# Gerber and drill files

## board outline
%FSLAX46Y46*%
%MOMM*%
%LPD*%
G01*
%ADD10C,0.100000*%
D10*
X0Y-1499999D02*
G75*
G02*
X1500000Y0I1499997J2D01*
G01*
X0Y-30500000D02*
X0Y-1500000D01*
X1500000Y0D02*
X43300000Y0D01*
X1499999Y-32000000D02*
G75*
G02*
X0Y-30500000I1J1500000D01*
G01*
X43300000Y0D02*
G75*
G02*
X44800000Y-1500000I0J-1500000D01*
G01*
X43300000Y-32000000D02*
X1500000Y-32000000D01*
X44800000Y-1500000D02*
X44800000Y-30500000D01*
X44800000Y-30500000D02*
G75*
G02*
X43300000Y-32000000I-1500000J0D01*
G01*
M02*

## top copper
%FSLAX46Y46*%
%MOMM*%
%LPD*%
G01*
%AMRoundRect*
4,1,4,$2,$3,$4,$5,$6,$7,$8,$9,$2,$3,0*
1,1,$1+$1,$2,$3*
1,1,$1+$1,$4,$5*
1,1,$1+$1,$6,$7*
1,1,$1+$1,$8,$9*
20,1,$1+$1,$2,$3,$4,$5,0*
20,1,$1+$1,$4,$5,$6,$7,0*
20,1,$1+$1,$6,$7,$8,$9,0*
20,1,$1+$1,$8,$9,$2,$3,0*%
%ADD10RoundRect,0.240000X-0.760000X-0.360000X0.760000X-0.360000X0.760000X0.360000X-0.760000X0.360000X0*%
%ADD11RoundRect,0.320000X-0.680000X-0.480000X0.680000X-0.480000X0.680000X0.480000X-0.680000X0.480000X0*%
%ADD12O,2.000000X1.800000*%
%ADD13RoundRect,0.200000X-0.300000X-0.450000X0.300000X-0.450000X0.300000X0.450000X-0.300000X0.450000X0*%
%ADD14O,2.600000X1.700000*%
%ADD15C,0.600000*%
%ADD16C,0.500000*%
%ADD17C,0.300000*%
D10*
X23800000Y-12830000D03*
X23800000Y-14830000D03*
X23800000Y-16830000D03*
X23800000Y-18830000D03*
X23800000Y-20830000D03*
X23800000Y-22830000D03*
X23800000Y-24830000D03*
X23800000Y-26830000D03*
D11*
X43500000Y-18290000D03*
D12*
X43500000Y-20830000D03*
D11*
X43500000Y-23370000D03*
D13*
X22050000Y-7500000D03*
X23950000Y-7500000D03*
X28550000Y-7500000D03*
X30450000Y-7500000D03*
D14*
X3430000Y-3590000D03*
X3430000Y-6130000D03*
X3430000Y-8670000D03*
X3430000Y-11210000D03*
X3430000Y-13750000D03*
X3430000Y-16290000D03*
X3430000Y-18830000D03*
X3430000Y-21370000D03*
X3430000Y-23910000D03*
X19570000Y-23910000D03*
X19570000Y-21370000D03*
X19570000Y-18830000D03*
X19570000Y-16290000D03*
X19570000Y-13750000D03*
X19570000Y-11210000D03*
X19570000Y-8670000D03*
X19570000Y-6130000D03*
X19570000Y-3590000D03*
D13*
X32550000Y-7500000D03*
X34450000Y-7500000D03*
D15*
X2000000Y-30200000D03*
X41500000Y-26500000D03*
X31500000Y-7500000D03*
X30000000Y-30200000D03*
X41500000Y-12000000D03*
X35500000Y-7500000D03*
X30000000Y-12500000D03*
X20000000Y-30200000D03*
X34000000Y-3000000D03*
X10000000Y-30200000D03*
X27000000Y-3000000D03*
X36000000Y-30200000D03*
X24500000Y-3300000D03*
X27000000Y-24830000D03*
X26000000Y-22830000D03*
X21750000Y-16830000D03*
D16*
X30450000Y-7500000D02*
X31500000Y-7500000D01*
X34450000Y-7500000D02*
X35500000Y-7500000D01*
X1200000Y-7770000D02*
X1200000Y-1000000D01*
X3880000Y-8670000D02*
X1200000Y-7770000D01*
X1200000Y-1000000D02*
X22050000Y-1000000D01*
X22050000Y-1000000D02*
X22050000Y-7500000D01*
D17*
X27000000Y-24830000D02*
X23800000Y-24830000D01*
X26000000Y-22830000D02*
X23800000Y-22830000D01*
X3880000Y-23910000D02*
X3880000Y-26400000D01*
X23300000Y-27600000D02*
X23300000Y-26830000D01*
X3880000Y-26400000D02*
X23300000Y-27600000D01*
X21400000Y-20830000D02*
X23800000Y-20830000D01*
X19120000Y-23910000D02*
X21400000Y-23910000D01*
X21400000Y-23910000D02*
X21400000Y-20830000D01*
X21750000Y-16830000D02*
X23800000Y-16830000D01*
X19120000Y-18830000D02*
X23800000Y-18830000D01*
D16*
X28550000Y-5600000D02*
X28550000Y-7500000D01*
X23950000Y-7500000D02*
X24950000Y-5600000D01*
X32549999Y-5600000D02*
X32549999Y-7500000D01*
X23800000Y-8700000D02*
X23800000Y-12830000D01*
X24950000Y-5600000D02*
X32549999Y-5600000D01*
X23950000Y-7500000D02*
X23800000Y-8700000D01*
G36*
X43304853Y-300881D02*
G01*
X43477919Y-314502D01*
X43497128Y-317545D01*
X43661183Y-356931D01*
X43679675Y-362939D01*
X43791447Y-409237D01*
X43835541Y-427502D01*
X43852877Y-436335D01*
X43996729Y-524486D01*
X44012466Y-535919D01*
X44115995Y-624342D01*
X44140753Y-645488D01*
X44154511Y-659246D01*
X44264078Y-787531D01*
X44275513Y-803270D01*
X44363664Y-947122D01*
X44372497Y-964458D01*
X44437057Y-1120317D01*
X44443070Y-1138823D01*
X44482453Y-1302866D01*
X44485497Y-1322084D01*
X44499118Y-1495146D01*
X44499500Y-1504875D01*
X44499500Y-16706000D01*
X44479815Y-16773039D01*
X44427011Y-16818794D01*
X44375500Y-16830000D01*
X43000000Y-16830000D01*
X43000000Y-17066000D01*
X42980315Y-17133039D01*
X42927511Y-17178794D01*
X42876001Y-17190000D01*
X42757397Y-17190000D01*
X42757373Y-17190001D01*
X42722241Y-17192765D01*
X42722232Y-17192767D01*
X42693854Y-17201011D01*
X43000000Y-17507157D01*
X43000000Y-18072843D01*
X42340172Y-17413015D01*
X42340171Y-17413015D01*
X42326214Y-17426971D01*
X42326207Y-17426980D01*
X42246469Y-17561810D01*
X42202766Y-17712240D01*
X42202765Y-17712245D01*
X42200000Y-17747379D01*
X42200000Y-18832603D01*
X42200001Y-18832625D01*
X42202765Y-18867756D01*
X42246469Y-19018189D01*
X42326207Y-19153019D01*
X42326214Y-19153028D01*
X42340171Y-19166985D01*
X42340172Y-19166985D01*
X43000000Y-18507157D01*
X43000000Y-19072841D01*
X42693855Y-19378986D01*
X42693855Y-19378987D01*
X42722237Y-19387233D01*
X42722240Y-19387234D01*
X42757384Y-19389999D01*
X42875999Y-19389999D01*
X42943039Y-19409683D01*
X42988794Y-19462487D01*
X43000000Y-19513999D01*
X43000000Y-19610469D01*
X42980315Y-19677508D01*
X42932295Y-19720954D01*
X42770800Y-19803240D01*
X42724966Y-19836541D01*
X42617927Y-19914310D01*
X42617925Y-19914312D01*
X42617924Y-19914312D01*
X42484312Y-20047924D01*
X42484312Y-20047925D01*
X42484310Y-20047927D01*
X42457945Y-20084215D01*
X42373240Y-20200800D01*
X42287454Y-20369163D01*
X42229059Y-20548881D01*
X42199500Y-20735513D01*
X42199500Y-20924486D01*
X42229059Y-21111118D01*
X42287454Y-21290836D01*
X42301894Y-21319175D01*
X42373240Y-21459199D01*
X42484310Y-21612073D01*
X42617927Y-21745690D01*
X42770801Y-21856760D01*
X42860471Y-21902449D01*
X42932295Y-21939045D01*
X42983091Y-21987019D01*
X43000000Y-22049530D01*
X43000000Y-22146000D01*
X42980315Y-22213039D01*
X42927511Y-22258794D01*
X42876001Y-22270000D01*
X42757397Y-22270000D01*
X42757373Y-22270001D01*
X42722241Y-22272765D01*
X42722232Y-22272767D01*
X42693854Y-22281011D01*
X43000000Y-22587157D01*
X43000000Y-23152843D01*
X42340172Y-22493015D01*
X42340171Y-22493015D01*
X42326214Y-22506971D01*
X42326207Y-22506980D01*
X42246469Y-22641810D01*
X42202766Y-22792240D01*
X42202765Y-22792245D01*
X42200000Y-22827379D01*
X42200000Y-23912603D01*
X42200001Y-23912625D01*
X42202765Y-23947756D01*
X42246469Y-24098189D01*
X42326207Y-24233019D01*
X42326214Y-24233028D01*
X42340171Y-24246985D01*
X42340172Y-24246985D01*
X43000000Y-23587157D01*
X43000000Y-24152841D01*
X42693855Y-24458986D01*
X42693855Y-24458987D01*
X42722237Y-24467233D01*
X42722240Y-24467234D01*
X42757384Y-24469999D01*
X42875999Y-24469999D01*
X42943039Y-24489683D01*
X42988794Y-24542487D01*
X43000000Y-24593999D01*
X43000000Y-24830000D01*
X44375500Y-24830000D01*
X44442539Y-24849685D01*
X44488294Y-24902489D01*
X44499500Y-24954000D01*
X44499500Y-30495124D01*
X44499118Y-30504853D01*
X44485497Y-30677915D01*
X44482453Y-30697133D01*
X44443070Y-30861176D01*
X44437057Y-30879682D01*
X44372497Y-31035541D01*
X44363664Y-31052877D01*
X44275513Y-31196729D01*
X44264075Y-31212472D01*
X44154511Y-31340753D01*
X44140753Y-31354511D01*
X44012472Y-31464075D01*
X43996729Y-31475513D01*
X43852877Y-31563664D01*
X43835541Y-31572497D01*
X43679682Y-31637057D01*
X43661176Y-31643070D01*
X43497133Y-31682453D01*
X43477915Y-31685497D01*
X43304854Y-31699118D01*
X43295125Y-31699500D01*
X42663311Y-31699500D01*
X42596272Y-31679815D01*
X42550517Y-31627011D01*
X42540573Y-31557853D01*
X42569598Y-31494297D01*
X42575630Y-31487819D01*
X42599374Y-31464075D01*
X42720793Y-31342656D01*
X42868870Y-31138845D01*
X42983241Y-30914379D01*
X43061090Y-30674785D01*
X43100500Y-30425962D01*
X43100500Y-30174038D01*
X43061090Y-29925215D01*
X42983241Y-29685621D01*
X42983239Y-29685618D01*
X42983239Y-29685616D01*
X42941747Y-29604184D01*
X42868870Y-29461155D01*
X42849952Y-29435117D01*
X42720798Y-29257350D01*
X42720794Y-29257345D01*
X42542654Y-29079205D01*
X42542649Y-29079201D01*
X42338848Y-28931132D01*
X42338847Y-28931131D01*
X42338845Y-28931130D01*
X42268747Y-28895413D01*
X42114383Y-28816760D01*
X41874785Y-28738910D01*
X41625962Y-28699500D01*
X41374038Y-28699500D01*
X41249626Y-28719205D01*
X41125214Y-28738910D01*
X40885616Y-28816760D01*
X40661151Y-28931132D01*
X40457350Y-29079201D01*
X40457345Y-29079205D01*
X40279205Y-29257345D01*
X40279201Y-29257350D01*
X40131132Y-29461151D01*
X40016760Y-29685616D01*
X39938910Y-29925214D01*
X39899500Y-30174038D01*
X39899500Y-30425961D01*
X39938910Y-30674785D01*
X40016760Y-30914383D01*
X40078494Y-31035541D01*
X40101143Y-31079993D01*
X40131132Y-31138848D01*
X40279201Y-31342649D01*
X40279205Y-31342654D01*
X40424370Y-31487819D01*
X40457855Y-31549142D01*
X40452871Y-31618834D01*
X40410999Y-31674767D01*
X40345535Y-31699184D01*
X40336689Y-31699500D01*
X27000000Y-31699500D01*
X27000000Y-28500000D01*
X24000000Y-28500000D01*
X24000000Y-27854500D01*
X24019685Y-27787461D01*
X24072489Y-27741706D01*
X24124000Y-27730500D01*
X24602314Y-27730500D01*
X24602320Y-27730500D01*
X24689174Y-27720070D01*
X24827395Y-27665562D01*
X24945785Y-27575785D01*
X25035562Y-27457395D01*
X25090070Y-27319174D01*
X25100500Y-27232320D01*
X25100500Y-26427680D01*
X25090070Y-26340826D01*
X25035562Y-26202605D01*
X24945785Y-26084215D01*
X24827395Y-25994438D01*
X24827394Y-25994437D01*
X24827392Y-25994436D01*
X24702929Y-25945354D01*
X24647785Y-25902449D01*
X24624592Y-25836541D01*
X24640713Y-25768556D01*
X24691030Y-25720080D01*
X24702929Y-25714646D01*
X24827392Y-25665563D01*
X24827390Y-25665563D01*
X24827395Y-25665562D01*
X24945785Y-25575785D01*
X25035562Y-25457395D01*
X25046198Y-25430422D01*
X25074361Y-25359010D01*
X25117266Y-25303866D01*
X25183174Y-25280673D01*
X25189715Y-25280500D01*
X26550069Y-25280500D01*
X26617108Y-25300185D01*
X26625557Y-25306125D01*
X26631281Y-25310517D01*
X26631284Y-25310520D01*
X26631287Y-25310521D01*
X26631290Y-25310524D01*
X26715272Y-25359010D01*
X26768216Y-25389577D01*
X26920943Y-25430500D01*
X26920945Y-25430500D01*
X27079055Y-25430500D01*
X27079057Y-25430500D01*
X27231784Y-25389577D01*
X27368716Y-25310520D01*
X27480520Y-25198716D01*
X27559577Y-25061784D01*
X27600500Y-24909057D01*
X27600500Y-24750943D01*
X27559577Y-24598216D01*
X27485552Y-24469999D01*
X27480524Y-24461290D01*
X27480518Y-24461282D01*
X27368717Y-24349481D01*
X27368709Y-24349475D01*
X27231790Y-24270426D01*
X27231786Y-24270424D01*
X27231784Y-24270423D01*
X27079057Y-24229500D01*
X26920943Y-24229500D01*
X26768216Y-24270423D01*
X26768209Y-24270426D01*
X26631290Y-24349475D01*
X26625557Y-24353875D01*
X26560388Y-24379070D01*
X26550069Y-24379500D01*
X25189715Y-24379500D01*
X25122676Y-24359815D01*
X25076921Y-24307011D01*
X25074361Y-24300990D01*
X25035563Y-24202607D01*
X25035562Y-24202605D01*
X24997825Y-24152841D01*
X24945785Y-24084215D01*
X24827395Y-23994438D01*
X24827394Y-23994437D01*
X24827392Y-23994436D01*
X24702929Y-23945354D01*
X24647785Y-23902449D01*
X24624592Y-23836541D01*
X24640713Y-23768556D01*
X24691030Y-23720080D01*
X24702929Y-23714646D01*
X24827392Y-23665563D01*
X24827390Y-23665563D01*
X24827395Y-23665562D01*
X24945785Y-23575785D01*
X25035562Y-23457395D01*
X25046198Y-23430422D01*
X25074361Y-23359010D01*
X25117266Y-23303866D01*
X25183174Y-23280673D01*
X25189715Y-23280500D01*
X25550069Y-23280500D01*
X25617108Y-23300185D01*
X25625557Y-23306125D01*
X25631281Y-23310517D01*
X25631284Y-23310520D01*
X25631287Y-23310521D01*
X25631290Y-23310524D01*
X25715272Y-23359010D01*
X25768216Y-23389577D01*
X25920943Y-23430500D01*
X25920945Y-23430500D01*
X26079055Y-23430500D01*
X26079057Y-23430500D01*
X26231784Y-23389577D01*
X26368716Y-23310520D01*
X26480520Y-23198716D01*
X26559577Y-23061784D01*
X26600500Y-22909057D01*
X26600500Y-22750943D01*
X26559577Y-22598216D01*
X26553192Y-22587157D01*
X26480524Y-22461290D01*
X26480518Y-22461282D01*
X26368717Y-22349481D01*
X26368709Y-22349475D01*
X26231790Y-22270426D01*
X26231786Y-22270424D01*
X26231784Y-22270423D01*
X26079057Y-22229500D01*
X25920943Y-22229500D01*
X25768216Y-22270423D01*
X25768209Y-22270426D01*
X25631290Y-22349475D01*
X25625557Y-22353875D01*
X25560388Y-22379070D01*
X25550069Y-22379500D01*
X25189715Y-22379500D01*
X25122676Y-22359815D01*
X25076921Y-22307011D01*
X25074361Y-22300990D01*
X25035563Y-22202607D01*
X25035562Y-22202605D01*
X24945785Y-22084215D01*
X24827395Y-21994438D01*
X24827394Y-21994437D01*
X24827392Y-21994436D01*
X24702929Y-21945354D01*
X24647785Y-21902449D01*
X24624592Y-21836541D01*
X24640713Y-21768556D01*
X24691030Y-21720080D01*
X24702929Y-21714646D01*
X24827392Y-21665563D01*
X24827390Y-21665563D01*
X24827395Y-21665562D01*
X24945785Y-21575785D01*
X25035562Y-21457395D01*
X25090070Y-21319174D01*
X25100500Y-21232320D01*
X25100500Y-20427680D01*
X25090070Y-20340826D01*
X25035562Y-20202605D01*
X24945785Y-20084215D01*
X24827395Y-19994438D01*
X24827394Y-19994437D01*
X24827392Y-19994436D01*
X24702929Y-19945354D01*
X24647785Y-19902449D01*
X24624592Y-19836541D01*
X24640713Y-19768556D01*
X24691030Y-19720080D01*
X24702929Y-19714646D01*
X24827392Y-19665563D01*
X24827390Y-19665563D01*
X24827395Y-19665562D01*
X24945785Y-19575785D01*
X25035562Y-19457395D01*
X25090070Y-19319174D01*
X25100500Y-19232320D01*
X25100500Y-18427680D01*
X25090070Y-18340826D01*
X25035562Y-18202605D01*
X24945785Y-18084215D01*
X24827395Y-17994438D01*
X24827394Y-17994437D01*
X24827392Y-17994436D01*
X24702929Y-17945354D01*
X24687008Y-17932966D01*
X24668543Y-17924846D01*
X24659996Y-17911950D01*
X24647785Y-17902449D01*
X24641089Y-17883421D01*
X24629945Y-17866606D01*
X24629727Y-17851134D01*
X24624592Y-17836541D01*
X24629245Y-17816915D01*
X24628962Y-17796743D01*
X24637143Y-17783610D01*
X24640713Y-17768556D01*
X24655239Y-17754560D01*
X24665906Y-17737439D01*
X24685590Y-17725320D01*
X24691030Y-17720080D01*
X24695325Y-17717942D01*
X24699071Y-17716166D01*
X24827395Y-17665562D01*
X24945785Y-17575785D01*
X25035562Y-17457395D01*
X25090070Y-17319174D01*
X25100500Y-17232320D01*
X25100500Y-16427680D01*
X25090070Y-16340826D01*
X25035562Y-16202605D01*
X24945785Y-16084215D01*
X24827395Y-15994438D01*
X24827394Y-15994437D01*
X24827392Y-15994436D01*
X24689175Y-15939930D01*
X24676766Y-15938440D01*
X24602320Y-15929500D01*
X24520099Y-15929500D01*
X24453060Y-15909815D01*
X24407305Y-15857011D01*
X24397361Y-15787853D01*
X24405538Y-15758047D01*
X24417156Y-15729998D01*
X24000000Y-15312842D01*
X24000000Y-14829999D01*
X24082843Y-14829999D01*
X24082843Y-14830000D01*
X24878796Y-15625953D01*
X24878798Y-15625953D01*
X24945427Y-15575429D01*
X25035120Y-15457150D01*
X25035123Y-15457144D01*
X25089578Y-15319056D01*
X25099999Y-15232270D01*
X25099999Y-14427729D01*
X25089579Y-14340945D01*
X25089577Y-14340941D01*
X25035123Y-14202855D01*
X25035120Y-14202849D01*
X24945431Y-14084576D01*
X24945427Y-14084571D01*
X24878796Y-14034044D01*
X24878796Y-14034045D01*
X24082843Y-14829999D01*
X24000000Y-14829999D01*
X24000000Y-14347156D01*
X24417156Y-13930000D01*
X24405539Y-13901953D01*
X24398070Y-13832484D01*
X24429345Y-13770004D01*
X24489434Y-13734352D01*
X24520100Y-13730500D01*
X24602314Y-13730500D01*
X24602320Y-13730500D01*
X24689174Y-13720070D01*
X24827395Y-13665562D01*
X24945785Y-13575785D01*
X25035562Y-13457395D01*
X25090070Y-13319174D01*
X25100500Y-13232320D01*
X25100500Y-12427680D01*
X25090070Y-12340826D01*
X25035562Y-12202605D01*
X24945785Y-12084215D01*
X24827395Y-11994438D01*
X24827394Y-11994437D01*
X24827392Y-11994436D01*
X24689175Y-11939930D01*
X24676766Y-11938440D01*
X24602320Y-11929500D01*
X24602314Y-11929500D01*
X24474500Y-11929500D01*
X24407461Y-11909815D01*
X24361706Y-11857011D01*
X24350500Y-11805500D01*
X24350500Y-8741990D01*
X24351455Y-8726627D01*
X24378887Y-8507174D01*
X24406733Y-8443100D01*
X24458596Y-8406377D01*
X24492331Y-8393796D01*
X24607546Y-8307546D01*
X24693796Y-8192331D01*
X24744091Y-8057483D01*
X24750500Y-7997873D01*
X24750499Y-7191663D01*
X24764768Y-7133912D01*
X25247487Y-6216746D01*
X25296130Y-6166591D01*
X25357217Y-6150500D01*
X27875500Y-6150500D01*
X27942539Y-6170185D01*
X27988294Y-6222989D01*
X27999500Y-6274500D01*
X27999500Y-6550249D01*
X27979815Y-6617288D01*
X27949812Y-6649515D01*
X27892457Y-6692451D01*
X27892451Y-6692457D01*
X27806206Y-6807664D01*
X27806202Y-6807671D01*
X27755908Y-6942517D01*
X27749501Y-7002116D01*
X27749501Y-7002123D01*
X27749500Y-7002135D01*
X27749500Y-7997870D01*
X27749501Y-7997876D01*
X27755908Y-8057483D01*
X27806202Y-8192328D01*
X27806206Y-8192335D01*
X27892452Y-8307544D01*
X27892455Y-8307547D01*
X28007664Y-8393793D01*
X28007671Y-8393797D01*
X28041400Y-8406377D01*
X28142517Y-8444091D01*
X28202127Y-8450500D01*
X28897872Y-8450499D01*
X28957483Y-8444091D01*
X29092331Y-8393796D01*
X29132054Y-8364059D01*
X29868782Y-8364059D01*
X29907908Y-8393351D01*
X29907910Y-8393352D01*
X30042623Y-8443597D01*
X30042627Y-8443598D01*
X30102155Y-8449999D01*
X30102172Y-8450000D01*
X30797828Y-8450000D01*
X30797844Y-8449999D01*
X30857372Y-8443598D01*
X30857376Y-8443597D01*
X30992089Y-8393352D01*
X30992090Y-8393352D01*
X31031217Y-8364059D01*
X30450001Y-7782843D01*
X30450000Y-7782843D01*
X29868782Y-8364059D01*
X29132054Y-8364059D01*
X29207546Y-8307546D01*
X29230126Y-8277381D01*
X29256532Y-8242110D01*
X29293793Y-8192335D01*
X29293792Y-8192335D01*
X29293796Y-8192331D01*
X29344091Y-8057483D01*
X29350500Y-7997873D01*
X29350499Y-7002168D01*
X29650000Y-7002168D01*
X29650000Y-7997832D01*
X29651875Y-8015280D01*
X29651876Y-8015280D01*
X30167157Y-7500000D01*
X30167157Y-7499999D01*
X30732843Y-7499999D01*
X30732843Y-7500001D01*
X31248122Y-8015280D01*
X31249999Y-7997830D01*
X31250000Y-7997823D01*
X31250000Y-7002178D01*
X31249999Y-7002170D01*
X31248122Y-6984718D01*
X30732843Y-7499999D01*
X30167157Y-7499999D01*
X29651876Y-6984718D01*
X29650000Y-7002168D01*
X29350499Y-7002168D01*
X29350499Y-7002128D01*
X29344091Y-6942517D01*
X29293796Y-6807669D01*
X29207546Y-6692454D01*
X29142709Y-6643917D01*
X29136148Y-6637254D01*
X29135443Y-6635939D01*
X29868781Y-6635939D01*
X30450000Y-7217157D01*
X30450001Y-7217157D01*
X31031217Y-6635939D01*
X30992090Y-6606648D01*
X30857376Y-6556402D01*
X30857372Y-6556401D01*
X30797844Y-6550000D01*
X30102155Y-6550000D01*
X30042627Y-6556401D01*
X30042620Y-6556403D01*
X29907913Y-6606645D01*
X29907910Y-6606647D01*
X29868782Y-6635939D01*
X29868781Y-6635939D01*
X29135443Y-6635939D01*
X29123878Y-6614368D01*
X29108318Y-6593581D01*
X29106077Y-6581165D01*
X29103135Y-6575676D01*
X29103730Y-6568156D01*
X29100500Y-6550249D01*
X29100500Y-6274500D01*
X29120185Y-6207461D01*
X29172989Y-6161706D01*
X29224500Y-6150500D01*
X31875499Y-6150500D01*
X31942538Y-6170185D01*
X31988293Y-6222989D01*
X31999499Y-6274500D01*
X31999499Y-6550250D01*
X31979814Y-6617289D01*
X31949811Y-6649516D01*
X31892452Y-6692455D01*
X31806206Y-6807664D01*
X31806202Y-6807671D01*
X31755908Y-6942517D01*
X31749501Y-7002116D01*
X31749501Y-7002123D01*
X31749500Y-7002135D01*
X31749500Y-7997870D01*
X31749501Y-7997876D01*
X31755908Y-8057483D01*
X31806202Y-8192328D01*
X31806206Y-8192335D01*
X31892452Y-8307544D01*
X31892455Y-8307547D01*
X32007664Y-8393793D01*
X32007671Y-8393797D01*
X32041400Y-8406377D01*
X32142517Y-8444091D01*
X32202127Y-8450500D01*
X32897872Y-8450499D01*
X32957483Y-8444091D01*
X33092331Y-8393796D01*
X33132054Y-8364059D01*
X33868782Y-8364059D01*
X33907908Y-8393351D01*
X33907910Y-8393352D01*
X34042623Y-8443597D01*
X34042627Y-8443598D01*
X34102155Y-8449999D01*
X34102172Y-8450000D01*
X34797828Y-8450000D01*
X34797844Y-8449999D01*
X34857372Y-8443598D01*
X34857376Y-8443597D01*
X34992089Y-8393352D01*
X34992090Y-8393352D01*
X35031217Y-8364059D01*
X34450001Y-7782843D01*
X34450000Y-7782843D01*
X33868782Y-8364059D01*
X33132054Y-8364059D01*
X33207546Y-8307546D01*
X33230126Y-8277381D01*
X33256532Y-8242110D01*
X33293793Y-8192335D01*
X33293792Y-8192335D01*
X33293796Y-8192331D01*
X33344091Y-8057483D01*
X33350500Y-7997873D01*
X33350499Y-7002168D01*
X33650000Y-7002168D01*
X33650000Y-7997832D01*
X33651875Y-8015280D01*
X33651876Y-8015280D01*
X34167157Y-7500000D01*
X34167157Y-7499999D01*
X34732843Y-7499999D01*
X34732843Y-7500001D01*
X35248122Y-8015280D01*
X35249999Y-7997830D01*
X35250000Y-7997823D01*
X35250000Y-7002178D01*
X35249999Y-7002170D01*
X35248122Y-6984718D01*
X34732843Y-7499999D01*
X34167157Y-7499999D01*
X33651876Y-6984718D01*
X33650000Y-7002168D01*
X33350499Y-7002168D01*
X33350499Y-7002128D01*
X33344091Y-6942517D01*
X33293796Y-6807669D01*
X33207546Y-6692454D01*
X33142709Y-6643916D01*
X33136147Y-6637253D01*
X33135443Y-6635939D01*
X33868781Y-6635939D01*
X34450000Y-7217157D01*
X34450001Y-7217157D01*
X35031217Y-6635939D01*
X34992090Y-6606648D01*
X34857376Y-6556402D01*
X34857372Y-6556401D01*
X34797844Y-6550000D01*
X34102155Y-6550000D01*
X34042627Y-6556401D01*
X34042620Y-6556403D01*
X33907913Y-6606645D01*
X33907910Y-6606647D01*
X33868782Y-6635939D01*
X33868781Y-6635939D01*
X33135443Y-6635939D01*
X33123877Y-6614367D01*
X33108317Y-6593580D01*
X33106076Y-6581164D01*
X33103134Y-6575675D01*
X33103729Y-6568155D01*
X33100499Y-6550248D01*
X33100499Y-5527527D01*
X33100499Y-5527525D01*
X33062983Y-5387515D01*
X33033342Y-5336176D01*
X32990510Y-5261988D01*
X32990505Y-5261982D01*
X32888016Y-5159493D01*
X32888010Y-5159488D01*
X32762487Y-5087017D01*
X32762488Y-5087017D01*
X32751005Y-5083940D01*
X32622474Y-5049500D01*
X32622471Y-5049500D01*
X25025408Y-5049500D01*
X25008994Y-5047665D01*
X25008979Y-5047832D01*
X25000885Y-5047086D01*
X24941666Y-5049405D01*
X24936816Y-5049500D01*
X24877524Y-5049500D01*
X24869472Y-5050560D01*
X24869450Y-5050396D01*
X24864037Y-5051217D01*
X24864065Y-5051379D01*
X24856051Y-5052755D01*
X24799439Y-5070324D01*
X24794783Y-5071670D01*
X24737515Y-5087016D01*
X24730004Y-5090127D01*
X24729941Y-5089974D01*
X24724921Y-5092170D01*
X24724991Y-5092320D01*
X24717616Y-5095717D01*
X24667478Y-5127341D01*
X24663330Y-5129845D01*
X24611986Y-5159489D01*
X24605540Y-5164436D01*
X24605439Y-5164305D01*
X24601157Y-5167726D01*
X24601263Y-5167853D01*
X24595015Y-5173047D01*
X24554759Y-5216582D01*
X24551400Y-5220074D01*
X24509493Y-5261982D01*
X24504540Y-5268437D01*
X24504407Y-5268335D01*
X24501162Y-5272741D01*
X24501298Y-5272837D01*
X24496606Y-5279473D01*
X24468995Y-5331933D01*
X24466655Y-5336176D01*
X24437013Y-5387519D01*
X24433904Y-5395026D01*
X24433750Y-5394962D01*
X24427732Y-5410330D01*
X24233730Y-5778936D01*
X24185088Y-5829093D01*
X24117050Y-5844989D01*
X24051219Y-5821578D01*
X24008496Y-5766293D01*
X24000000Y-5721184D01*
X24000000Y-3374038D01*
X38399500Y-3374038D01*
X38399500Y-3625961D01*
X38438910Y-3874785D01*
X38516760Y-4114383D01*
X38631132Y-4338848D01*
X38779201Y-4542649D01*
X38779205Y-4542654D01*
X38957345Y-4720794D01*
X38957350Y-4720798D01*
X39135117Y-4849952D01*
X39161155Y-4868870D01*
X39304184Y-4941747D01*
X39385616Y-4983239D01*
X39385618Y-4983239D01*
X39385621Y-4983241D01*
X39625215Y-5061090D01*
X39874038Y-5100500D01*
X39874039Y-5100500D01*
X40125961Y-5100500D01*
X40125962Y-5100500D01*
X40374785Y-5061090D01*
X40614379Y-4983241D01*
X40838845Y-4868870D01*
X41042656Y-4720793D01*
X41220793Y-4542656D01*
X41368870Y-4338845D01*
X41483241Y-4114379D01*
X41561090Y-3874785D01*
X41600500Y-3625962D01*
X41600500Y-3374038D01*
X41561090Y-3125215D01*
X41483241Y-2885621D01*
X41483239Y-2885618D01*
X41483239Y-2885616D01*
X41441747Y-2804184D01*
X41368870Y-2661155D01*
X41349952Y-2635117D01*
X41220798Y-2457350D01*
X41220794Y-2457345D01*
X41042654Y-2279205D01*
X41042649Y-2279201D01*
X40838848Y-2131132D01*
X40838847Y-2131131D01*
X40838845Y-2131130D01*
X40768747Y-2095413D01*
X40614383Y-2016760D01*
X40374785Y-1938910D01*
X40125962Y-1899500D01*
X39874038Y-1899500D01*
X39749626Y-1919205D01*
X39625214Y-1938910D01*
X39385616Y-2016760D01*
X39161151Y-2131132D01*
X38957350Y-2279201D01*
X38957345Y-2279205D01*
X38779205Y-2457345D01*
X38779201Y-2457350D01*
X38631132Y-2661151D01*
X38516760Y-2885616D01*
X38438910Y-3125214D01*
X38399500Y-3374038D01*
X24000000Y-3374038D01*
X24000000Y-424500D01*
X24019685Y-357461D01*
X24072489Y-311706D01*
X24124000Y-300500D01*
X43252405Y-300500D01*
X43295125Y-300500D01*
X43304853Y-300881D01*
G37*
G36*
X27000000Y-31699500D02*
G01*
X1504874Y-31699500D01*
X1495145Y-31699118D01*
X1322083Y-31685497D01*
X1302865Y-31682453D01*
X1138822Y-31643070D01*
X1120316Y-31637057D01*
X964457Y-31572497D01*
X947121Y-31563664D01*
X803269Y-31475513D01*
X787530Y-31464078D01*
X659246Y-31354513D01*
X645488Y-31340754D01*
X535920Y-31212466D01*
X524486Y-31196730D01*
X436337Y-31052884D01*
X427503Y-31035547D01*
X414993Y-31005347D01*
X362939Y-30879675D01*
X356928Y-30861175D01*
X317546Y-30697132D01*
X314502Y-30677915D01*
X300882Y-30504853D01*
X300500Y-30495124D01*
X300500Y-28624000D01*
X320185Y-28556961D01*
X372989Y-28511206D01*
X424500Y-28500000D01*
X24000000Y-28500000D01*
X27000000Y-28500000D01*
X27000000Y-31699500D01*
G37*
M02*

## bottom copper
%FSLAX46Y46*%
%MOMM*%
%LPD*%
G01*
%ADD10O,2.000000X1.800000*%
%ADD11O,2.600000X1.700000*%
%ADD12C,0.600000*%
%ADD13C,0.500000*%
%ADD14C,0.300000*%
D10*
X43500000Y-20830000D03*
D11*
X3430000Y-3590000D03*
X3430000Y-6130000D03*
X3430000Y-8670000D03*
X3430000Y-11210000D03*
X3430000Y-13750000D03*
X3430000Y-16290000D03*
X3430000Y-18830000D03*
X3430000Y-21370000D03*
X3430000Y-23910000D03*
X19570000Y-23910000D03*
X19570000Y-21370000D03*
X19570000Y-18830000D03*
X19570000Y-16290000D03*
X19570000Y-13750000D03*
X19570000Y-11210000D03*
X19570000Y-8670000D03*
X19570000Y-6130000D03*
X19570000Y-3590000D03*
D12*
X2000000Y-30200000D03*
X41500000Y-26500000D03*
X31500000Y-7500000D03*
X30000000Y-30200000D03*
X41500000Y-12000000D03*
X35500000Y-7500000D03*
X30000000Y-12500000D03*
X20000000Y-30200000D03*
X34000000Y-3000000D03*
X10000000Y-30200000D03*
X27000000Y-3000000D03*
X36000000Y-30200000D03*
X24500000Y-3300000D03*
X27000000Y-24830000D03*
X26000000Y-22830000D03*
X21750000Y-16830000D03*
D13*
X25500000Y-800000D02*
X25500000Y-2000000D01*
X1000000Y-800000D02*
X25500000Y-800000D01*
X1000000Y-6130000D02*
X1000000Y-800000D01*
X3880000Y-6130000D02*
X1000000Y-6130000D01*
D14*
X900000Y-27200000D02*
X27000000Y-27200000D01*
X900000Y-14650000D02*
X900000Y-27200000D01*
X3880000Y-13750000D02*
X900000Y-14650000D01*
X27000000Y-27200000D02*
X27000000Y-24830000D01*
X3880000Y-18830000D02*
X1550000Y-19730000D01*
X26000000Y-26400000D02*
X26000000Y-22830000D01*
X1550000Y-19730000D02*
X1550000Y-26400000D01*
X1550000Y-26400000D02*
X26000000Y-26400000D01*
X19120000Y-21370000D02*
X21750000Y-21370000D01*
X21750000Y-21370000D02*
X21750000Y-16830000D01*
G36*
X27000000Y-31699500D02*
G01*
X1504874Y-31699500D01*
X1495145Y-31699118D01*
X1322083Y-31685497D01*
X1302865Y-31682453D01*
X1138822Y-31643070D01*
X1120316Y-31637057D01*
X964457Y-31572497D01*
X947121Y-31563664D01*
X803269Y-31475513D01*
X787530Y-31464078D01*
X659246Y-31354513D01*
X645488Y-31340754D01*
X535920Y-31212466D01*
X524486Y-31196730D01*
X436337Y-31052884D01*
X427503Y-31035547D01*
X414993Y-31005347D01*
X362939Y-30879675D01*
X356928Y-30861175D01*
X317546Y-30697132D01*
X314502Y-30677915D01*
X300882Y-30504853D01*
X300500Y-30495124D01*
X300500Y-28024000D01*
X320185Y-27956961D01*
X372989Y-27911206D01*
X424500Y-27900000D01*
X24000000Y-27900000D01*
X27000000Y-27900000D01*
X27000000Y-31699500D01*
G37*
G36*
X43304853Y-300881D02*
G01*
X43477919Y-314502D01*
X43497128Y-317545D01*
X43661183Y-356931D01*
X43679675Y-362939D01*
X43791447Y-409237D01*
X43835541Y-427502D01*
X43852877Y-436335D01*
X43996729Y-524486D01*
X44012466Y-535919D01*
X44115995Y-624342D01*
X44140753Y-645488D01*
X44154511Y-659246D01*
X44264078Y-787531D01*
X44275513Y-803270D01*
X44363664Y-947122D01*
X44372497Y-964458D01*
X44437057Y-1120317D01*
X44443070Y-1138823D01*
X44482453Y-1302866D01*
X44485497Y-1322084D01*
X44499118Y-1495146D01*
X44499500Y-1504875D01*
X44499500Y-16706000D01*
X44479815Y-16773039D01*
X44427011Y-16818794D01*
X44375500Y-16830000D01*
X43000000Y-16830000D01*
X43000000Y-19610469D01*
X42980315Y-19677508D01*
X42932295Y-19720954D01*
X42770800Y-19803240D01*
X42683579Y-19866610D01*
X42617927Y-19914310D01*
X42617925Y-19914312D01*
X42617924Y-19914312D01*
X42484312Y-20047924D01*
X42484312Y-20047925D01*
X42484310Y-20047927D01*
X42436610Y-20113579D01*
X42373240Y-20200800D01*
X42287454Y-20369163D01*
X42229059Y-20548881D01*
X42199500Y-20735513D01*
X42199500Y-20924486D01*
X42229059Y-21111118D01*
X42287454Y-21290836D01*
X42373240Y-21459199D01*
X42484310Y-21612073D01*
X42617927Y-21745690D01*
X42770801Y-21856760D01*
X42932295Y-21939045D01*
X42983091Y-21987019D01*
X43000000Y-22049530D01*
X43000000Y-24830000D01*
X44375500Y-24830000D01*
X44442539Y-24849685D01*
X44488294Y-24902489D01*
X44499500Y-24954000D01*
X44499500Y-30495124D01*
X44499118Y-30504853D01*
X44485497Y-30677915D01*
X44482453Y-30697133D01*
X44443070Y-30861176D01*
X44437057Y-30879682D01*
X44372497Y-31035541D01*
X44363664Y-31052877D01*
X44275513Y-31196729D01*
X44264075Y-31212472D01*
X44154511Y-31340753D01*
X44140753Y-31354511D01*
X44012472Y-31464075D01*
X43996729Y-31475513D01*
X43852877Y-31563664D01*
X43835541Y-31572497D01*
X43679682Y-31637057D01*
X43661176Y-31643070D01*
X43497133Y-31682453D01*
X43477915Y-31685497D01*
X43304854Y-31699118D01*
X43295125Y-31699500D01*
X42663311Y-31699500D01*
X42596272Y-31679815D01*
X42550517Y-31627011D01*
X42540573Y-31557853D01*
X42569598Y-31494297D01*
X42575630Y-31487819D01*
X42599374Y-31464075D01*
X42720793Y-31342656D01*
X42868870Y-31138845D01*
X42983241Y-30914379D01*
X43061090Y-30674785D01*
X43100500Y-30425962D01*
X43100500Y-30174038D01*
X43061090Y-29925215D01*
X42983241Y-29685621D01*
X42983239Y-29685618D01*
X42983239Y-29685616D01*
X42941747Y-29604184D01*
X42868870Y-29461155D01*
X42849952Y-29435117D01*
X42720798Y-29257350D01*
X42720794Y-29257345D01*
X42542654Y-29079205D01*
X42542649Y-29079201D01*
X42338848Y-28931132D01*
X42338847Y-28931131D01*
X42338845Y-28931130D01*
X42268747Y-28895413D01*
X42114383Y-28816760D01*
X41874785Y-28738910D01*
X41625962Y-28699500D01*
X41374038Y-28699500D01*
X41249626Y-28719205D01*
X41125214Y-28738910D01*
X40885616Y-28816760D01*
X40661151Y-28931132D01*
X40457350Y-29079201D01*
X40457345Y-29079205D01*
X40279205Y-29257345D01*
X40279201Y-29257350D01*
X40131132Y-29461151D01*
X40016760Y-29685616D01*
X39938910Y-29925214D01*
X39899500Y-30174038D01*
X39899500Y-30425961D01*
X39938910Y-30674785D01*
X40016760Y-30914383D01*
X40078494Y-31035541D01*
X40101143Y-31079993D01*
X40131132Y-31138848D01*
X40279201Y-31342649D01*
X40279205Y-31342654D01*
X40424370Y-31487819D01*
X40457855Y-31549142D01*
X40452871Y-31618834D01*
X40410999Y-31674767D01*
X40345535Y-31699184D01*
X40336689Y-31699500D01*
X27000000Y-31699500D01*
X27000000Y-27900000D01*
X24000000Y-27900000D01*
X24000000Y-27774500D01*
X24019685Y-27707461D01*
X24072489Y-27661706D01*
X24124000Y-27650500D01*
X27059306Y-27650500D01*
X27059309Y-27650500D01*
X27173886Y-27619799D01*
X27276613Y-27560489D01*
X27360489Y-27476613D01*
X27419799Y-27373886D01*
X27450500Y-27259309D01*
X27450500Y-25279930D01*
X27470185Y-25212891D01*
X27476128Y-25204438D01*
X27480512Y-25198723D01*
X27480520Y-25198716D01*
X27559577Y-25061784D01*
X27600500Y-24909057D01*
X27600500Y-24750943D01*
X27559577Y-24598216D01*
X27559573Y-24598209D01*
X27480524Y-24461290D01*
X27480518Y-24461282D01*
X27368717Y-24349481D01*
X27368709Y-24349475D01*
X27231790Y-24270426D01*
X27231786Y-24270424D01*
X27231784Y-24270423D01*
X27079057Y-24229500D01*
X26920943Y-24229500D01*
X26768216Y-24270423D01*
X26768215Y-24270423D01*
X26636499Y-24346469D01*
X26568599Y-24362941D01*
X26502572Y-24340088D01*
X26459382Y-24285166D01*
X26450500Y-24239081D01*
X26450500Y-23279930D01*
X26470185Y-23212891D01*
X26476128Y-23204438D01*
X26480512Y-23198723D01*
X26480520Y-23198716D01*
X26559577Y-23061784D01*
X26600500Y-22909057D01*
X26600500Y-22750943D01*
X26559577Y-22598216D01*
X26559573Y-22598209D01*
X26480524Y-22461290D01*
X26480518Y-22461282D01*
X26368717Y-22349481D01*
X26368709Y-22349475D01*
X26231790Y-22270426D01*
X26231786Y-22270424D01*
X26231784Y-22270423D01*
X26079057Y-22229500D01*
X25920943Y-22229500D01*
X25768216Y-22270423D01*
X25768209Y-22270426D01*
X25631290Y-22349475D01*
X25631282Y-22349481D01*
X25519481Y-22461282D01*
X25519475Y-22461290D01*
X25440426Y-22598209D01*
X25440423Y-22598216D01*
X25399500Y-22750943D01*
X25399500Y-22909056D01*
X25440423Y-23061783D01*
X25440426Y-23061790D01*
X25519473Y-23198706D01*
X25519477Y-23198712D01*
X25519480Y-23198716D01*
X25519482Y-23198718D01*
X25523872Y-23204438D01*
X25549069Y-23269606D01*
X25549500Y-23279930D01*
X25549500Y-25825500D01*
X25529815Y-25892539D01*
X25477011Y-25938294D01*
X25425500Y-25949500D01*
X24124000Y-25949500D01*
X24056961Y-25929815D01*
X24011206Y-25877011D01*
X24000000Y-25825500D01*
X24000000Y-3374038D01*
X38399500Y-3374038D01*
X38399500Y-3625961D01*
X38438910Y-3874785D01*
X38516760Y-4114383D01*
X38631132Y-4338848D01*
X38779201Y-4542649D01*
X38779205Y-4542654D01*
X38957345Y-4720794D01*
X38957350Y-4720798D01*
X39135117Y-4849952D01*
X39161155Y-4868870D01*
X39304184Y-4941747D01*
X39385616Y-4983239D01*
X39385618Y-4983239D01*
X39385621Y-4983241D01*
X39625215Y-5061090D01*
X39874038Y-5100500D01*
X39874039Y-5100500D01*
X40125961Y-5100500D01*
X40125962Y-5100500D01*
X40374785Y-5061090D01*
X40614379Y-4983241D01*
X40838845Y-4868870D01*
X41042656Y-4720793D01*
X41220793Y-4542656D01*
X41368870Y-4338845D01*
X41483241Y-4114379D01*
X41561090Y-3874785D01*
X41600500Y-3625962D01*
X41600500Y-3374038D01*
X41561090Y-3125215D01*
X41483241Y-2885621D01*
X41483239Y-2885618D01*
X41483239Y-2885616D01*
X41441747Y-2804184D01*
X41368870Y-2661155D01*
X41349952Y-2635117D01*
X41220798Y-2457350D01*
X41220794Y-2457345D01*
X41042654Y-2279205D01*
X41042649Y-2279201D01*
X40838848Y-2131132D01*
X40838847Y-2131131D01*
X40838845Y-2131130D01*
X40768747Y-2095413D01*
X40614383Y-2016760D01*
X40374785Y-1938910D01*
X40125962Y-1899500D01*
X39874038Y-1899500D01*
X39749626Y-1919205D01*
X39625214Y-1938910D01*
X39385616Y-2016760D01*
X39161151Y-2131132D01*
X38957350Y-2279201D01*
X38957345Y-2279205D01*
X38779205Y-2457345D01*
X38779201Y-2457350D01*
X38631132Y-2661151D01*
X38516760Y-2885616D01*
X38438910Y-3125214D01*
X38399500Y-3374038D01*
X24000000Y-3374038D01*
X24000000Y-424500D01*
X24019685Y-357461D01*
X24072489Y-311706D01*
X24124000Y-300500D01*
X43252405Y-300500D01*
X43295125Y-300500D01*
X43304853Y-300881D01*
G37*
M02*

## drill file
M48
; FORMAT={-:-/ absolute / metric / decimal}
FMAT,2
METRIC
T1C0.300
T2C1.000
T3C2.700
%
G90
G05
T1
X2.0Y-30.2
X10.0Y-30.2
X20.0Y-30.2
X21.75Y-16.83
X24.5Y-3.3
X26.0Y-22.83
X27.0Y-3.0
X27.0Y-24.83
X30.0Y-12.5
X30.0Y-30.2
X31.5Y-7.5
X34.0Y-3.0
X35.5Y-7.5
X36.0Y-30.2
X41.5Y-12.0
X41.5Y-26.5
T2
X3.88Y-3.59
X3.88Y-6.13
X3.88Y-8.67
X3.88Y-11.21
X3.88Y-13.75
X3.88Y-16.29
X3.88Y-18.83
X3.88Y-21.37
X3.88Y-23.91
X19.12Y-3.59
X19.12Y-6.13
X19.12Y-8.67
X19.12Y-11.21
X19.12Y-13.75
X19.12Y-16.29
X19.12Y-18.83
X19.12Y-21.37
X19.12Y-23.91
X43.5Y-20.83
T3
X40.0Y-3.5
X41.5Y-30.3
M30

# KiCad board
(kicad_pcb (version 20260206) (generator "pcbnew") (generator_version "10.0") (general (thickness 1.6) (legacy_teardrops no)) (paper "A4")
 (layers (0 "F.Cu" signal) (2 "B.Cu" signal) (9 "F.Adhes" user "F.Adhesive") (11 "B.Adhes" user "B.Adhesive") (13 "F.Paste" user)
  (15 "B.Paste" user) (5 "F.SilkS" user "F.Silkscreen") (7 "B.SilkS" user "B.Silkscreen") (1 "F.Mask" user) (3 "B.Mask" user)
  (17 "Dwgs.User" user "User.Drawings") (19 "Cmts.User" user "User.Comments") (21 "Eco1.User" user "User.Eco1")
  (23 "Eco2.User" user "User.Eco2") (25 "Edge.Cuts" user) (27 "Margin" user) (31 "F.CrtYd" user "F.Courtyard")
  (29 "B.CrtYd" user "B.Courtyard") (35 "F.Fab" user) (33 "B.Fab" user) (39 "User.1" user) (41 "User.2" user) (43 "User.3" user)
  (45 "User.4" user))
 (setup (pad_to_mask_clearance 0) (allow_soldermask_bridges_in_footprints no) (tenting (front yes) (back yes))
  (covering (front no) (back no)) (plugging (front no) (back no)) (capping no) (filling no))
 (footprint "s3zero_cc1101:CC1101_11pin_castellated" (layer "F.Cu") (at 33.65 19.83)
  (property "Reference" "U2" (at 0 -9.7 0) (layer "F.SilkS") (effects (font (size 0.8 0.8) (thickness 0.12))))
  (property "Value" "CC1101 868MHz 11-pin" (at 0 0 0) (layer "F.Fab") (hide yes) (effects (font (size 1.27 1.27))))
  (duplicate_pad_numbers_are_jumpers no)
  (pad "1" smd roundrect (at -9.85 -7) (size 2 1.2) (layers "F.Cu" "F.Mask" "F.Paste") (roundrect_rratio 0.2) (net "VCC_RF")
   (thermal_bridge_angle 45))
  (pad "2" smd roundrect (at -9.85 -5) (size 2 1.2) (layers "F.Cu" "F.Mask" "F.Paste") (roundrect_rratio 0.2) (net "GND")
   (thermal_bridge_angle 45))
  (pad "3" smd roundrect (at -9.85 -3) (size 2 1.2) (layers "F.Cu" "F.Mask" "F.Paste") (roundrect_rratio 0.2) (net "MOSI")
   (thermal_bridge_angle 45))
  (pad "4" smd roundrect (at -9.85 -1) (size 2 1.2) (layers "F.Cu" "F.Mask" "F.Paste") (roundrect_rratio 0.2) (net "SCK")
   (thermal_bridge_angle 45))
  (pad "5" smd roundrect (at -9.85 1) (size 2 1.2) (layers "F.Cu" "F.Mask" "F.Paste") (roundrect_rratio 0.2) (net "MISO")
   (thermal_bridge_angle 45))
  (pad "6" smd roundrect (at -9.85 3) (size 2 1.2) (layers "F.Cu" "F.Mask" "F.Paste") (roundrect_rratio 0.2) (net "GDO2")
   (thermal_bridge_angle 45))
  (pad "7" smd roundrect (at -9.85 5) (size 2 1.2) (layers "F.Cu" "F.Mask" "F.Paste") (roundrect_rratio 0.2) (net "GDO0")
   (thermal_bridge_angle 45))
  (pad "8" smd roundrect (at -9.85 7) (size 2 1.2) (layers "F.Cu" "F.Mask" "F.Paste") (roundrect_rratio 0.2) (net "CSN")
   (thermal_bridge_angle 45))
  (pad "9" smd roundrect (at 9.85 -1.54) (size 2 1.6) (layers "F.Cu" "F.Mask" "F.Paste") (roundrect_rratio 0.2) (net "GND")
   (thermal_bridge_angle 45))
  (pad "10" thru_hole oval (at 9.85 1) (size 2 1.8) (drill 1) (layers "*.Cu" "*.Mask") (remove_unused_layers no)
   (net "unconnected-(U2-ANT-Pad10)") (thermal_bridge_angle 45))
  (pad "11" smd roundrect (at 9.85 3.54) (size 2 1.6) (layers "F.Cu" "F.Mask" "F.Paste") (roundrect_rratio 0.2) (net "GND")
   (thermal_bridge_angle 45)))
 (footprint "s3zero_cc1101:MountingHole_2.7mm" (layer "F.Cu") (at 40 3.5)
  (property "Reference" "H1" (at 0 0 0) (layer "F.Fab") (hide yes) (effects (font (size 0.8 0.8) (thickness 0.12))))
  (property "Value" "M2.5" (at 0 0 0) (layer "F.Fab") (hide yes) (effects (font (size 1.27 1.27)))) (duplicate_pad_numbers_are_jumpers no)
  (pad "" np_thru_hole circle (at 0 0) (size 2.7 2.7) (drill 2.7) (layers "*.Cu" "*.Mask")))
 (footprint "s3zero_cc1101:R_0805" (layer "F.Cu") (at 23 7.5)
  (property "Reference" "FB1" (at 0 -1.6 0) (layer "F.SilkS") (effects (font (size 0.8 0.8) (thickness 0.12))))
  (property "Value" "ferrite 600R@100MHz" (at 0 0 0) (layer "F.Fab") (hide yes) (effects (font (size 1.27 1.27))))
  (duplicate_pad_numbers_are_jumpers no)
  (pad "1" smd roundrect (at -0.95 0) (size 1 1.3) (layers "F.Cu" "F.Mask" "F.Paste") (roundrect_rratio 0.2) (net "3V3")
   (thermal_bridge_angle 45))
  (pad "2" smd roundrect (at 0.95 0) (size 1 1.3) (layers "F.Cu" "F.Mask" "F.Paste") (roundrect_rratio 0.2) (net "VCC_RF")
   (thermal_bridge_angle 45)))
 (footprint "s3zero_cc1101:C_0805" (layer "F.Cu") (at 29.5 7.5)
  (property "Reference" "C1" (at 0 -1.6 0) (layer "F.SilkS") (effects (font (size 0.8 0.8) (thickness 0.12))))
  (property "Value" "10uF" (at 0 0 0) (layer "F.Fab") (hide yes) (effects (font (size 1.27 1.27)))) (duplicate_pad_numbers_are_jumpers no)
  (pad "1" smd roundrect (at -0.95 0) (size 1 1.3) (layers "F.Cu" "F.Mask" "F.Paste") (roundrect_rratio 0.2) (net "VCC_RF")
   (thermal_bridge_angle 45))
  (pad "2" smd roundrect (at 0.95 0) (size 1 1.3) (layers "F.Cu" "F.Mask" "F.Paste") (roundrect_rratio 0.2) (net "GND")
   (thermal_bridge_angle 45)))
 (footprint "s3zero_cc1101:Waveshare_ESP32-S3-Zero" (layer "F.Cu") (at 2.5 2)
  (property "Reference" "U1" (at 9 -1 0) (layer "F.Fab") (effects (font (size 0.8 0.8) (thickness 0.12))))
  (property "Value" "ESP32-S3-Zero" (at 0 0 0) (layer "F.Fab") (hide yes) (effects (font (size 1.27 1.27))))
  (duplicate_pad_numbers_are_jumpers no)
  (pad "1" thru_hole oval (at 1.38 1.59) (size 2.6 1.7) (drill 1 (offset -0.45 0)) (layers "*.Cu" "*.Mask") (remove_unused_layers no)
   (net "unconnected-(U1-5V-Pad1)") (thermal_bridge_angle 45))
  (pad "2" thru_hole oval (at 1.38 4.13) (size 2.6 1.7) (drill 1 (offset -0.45 0)) (layers "*.Cu" "*.Mask") (remove_unused_layers no)
   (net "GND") (thermal_bridge_angle 45))
  (pad "3" thru_hole oval (at 1.38 6.67) (size 2.6 1.7) (drill 1 (offset -0.45 0)) (layers "*.Cu" "*.Mask") (remove_unused_layers no)
   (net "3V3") (thermal_bridge_angle 45))
  (pad "4" thru_hole oval (at 1.38 9.21) (size 2.6 1.7) (drill 1 (offset -0.45 0)) (layers "*.Cu" "*.Mask") (remove_unused_layers no)
   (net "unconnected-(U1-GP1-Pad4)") (thermal_bridge_angle 45))
  (pad "5" thru_hole oval (at 1.38 11.75) (size 2.6 1.7) (drill 1 (offset -0.45 0)) (layers "*.Cu" "*.Mask") (remove_unused_layers no)
   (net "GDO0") (thermal_bridge_angle 45))
  (pad "6" thru_hole oval (at 1.38 14.29) (size 2.6 1.7) (drill 1 (offset -0.45 0)) (layers "*.Cu" "*.Mask") (remove_unused_layers no)
   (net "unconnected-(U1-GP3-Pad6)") (thermal_bridge_angle 45))
  (pad "7" thru_hole oval (at 1.38 16.83) (size 2.6 1.7) (drill 1 (offset -0.45 0)) (layers "*.Cu" "*.Mask") (remove_unused_layers no)
   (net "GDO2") (thermal_bridge_angle 45))
  (pad "8" thru_hole oval (at 1.38 19.37) (size 2.6 1.7) (drill 1 (offset -0.45 0)) (layers "*.Cu" "*.Mask") (remove_unused_layers no)
   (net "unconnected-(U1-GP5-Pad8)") (thermal_bridge_angle 45))
  (pad "9" thru_hole oval (at 1.38 21.91) (size 2.6 1.7) (drill 1 (offset -0.45 0)) (layers "*.Cu" "*.Mask") (remove_unused_layers no)
   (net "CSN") (thermal_bridge_angle 45))
  (pad "10" thru_hole oval (at 16.62 21.91) (size 2.6 1.7) (drill 1 (offset 0.45 0)) (layers "*.Cu" "*.Mask") (remove_unused_layers no)
   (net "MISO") (thermal_bridge_angle 45))
  (pad "11" thru_hole oval (at 16.62 19.37) (size 2.6 1.7) (drill 1 (offset 0.45 0)) (layers "*.Cu" "*.Mask") (remove_unused_layers no)
   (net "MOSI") (thermal_bridge_angle 45))
  (pad "12" thru_hole oval (at 16.62 16.83) (size 2.6 1.7) (drill 1 (offset 0.45 0)) (layers "*.Cu" "*.Mask") (remove_unused_layers no)
   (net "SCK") (thermal_bridge_angle 45))
  (pad "13" thru_hole oval (at 16.62 14.29) (size 2.6 1.7) (drill 1 (offset 0.45 0)) (layers "*.Cu" "*.Mask") (remove_unused_layers no)
   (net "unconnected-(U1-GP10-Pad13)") (thermal_bridge_angle 45))
  (pad "14" thru_hole oval (at 16.62 11.75) (size 2.6 1.7) (drill 1 (offset 0.45 0)) (layers "*.Cu" "*.Mask") (remove_unused_layers no)
   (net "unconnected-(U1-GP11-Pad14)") (thermal_bridge_angle 45))
  (pad "15" thru_hole oval (at 16.62 9.21) (size 2.6 1.7) (drill 1 (offset 0.45 0)) (layers "*.Cu" "*.Mask") (remove_unused_layers no)
   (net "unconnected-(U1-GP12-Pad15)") (thermal_bridge_angle 45))
  (pad "16" thru_hole oval (at 16.62 6.67) (size 2.6 1.7) (drill 1 (offset 0.45 0)) (layers "*.Cu" "*.Mask") (remove_unused_layers no)
   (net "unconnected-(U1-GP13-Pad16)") (thermal_bridge_angle 45))
  (pad "17" thru_hole oval (at 16.62 4.13) (size 2.6 1.7) (drill 1 (offset 0.45 0)) (layers "*.Cu" "*.Mask") (remove_unused_layers no)
   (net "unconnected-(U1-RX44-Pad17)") (thermal_bridge_angle 45))
  (pad "18" thru_hole oval (at 16.62 1.59) (size 2.6 1.7) (drill 1 (offset 0.45 0)) (layers "*.Cu" "*.Mask") (remove_unused_layers no)
   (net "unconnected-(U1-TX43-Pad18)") (thermal_bridge_angle 45)))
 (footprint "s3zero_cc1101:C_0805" (layer "F.Cu") (at 33.5 7.5)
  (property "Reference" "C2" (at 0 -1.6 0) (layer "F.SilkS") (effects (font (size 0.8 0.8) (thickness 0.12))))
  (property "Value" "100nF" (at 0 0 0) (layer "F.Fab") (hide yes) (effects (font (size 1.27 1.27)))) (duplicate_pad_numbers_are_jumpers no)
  (pad "1" smd roundrect (at -0.95 0) (size 1 1.3) (layers "F.Cu" "F.Mask" "F.Paste") (roundrect_rratio 0.2) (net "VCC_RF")
   (thermal_bridge_angle 45))
  (pad "2" smd roundrect (at 0.95 0) (size 1 1.3) (layers "F.Cu" "F.Mask" "F.Paste") (roundrect_rratio 0.2) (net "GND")
   (thermal_bridge_angle 45)))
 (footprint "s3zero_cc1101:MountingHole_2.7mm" (layer "F.Cu") (at 41.5 30.3)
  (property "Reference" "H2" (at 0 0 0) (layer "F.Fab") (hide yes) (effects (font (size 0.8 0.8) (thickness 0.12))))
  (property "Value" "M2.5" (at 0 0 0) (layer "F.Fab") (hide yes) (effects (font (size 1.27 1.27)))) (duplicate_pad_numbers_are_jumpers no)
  (pad "" np_thru_hole circle (at 0 0) (size 2.7 2.7) (drill 2.7) (layers "*.Cu" "*.Mask")))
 (gr_arc (start 0 1.499999) (mid 0.439339 0.439339) (end 1.5 0) (stroke (width 0.1) (type default)) (layer "Edge.Cuts"))
 (gr_line (start 0 30.5) (end 0 1.5) (stroke (width 0.1) (type default)) (layer "Edge.Cuts"))
 (gr_line (start 1.5 0) (end 43.3 0) (stroke (width 0.1) (type default)) (layer "Edge.Cuts"))
 (gr_arc (start 1.499999 32) (mid 0.439339 31.56066) (end 0 30.5) (stroke (width 0.1) (type default)) (layer "Edge.Cuts"))
 (gr_arc (start 43.3 0) (mid 44.36066 0.43934) (end 44.8 1.5) (stroke (width 0.1) (type default)) (layer "Edge.Cuts"))
 (gr_line (start 43.3 32) (end 1.5 32) (stroke (width 0.1) (type default)) (layer "Edge.Cuts"))
 (gr_line (start 44.8 1.5) (end 44.8 30.5) (stroke (width 0.1) (type default)) (layer "Edge.Cuts"))
 (gr_arc (start 44.8 30.5) (mid 44.36066 31.56066) (end 43.3 32) (stroke (width 0.1) (type default)) (layer "Edge.Cuts"))
 (segment (start 30.45 7.5) (end 31.5 7.5) (width 0.5) (layer "F.Cu") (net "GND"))
 (segment (start 34.45 7.5) (end 35.5 7.5) (width 0.5) (layer "F.Cu") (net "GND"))
 (via (at 2 30.2) (size 0.6) (drill 0.3) (layers "F.Cu" "B.Cu") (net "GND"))
 (via (at 41.5 26.5) (size 0.6) (drill 0.3) (layers "F.Cu" "B.Cu") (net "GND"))
 (via (at 31.5 7.5) (size 0.6) (drill 0.3) (layers "F.Cu" "B.Cu") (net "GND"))
 (via (at 30 30.2) (size 0.6) (drill 0.3) (layers "F.Cu" "B.Cu") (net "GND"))
 (via (at 41.5 12) (size 0.6) (drill 0.3) (layers "F.Cu" "B.Cu") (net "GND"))
 (via (at 35.5 7.5) (size 0.6) (drill 0.3) (layers "F.Cu" "B.Cu") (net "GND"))
 (via (at 30 12.5) (size 0.6) (drill 0.3) (layers "F.Cu" "B.Cu") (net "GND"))
 (via (at 20 30.2) (size 0.6) (drill 0.3) (layers "F.Cu" "B.Cu") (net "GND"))
 (via (at 34 3) (size 0.6) (drill 0.3) (layers "F.Cu" "B.Cu") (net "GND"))
 (via (at 10 30.2) (size 0.6) (drill 0.3) (layers "F.Cu" "B.Cu") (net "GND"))
 (via (at 27 3) (size 0.6) (drill 0.3) (layers "F.Cu" "B.Cu") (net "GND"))
 (via (at 36 30.2) (size 0.6) (drill 0.3) (layers "F.Cu" "B.Cu") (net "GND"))
 (via (at 24.5 3.3) (size 0.6) (drill 0.3) (layers "F.Cu" "B.Cu") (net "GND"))
 (segment (start 25.5 0.8) (end 25.5 2) (width 0.5) (layer "B.Cu") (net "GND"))
 (segment (start 1 0.8) (end 25.5 0.8) (width 0.5) (layer "B.Cu") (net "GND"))
 (segment (start 1 6.13) (end 1 0.8) (width 0.5) (layer "B.Cu") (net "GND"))
 (segment (start 3.88 6.13) (end 1 6.13) (width 0.5) (layer "B.Cu") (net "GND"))
 (segment (start 1.2 7.77) (end 1.2 1) (width 0.5) (layer "F.Cu") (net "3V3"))
 (segment (start 3.88 8.67) (end 1.2 7.77) (width 0.5) (layer "F.Cu") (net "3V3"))
 (segment (start 1.2 1) (end 22.05 1) (width 0.5) (layer "F.Cu") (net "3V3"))
 (segment (start 22.05 1) (end 22.05 7.5) (width 0.5) (layer "F.Cu") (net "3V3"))
 (segment (start 27 24.83) (end 23.8 24.83) (width 0.3) (layer "F.Cu") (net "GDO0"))
 (via (at 27 24.83) (size 0.6) (drill 0.3) (layers "F.Cu" "B.Cu") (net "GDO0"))
 (segment (start 0.9 27.2) (end 27 27.2) (width 0.3) (layer "B.Cu") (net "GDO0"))
 (segment (start 0.9 14.65) (end 0.9 27.2) (width 0.3) (layer "B.Cu") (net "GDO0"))
 (segment (start 3.88 13.75) (end 0.9 14.65) (width 0.3) (layer "B.Cu") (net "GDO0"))
 (segment (start 27 27.2) (end 27 24.83) (width 0.3) (layer "B.Cu") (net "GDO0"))
 (segment (start 26 22.83) (end 23.8 22.83) (width 0.3) (layer "F.Cu") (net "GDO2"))
 (via (at 26 22.83) (size 0.6) (drill 0.3) (layers "F.Cu" "B.Cu") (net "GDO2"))
 (segment (start 3.88 18.83) (end 1.55 19.73) (width 0.3) (layer "B.Cu") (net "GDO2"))
 (segment (start 26 26.4) (end 26 22.83) (width 0.3) (layer "B.Cu") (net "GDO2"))
 (segment (start 1.55 19.73) (end 1.55 26.4) (width 0.3) (layer "B.Cu") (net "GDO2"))
 (segment (start 1.55 26.4) (end 26 26.4) (width 0.3) (layer "B.Cu") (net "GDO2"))
 (segment (start 3.88 23.91) (end 3.88 26.4) (width 0.3) (layer "F.Cu") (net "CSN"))
 (segment (start 23.3 27.6) (end 23.3 26.83) (width 0.3) (layer "F.Cu") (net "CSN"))
 (segment (start 3.88 26.4) (end 23.3 27.6) (width 0.3) (layer "F.Cu") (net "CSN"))
 (segment (start 21.4 20.83) (end 23.8 20.83) (width 0.3) (layer "F.Cu") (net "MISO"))
 (segment (start 19.12 23.91) (end 21.4 23.91) (width 0.3) (layer "F.Cu") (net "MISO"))
 (segment (start 21.4 23.91) (end 21.4 20.83) (width 0.3) (layer "F.Cu") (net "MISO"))
 (segment (start 21.75 16.83) (end 23.8 16.83) (width 0.3) (layer "F.Cu") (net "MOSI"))
 (via (at 21.75 16.83) (size 0.6) (drill 0.3) (layers "F.Cu" "B.Cu") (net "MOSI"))
 (segment (start 19.12 21.37) (end 21.75 21.37) (width 0.3) (layer "B.Cu") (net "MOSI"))
 (segment (start 21.75 21.37) (end 21.75 16.83) (width 0.3) (layer "B.Cu") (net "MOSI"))
 (segment (start 19.12 18.83) (end 23.8 18.83) (width 0.3) (layer "F.Cu") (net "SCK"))
 (segment (start 28.55 5.6) (end 28.55 7.5) (width 0.5) (layer "F.Cu") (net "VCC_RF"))
 (segment (start 23.95 7.5) (end 24.95 5.6) (width 0.5) (layer "F.Cu") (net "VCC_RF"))
 (segment (start 32.549999 5.6) (end 32.549999 7.5) (width 0.5) (layer "F.Cu") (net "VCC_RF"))
 (segment (start 23.8 8.7) (end 23.8 12.83) (width 0.5) (layer "F.Cu") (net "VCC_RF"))
 (segment (start 24.95 5.6) (end 32.549999 5.6) (width 0.5) (layer "F.Cu") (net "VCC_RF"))
 (segment (start 23.95 7.5) (end 23.8 8.7) (width 0.5) (layer "F.Cu") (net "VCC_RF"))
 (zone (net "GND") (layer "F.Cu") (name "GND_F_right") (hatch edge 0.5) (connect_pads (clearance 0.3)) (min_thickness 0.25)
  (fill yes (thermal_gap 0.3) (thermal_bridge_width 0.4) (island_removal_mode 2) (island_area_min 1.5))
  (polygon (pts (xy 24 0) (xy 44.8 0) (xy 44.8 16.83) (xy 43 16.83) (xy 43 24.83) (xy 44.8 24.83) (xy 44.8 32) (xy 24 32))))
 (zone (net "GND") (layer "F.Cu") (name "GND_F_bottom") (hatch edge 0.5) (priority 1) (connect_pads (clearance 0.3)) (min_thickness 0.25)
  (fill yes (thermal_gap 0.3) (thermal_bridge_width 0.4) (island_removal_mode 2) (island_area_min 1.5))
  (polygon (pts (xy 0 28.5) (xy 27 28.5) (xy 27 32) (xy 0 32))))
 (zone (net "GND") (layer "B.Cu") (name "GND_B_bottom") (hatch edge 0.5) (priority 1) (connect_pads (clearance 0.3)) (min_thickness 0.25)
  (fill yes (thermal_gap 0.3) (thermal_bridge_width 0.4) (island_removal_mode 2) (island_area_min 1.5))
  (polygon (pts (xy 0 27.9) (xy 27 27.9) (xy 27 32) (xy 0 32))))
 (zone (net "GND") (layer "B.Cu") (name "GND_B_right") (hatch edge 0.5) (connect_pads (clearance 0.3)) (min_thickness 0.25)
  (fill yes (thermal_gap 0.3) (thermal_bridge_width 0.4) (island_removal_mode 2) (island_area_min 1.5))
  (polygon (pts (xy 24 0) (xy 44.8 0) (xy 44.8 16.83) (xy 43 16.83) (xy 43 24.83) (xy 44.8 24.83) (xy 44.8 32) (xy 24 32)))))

